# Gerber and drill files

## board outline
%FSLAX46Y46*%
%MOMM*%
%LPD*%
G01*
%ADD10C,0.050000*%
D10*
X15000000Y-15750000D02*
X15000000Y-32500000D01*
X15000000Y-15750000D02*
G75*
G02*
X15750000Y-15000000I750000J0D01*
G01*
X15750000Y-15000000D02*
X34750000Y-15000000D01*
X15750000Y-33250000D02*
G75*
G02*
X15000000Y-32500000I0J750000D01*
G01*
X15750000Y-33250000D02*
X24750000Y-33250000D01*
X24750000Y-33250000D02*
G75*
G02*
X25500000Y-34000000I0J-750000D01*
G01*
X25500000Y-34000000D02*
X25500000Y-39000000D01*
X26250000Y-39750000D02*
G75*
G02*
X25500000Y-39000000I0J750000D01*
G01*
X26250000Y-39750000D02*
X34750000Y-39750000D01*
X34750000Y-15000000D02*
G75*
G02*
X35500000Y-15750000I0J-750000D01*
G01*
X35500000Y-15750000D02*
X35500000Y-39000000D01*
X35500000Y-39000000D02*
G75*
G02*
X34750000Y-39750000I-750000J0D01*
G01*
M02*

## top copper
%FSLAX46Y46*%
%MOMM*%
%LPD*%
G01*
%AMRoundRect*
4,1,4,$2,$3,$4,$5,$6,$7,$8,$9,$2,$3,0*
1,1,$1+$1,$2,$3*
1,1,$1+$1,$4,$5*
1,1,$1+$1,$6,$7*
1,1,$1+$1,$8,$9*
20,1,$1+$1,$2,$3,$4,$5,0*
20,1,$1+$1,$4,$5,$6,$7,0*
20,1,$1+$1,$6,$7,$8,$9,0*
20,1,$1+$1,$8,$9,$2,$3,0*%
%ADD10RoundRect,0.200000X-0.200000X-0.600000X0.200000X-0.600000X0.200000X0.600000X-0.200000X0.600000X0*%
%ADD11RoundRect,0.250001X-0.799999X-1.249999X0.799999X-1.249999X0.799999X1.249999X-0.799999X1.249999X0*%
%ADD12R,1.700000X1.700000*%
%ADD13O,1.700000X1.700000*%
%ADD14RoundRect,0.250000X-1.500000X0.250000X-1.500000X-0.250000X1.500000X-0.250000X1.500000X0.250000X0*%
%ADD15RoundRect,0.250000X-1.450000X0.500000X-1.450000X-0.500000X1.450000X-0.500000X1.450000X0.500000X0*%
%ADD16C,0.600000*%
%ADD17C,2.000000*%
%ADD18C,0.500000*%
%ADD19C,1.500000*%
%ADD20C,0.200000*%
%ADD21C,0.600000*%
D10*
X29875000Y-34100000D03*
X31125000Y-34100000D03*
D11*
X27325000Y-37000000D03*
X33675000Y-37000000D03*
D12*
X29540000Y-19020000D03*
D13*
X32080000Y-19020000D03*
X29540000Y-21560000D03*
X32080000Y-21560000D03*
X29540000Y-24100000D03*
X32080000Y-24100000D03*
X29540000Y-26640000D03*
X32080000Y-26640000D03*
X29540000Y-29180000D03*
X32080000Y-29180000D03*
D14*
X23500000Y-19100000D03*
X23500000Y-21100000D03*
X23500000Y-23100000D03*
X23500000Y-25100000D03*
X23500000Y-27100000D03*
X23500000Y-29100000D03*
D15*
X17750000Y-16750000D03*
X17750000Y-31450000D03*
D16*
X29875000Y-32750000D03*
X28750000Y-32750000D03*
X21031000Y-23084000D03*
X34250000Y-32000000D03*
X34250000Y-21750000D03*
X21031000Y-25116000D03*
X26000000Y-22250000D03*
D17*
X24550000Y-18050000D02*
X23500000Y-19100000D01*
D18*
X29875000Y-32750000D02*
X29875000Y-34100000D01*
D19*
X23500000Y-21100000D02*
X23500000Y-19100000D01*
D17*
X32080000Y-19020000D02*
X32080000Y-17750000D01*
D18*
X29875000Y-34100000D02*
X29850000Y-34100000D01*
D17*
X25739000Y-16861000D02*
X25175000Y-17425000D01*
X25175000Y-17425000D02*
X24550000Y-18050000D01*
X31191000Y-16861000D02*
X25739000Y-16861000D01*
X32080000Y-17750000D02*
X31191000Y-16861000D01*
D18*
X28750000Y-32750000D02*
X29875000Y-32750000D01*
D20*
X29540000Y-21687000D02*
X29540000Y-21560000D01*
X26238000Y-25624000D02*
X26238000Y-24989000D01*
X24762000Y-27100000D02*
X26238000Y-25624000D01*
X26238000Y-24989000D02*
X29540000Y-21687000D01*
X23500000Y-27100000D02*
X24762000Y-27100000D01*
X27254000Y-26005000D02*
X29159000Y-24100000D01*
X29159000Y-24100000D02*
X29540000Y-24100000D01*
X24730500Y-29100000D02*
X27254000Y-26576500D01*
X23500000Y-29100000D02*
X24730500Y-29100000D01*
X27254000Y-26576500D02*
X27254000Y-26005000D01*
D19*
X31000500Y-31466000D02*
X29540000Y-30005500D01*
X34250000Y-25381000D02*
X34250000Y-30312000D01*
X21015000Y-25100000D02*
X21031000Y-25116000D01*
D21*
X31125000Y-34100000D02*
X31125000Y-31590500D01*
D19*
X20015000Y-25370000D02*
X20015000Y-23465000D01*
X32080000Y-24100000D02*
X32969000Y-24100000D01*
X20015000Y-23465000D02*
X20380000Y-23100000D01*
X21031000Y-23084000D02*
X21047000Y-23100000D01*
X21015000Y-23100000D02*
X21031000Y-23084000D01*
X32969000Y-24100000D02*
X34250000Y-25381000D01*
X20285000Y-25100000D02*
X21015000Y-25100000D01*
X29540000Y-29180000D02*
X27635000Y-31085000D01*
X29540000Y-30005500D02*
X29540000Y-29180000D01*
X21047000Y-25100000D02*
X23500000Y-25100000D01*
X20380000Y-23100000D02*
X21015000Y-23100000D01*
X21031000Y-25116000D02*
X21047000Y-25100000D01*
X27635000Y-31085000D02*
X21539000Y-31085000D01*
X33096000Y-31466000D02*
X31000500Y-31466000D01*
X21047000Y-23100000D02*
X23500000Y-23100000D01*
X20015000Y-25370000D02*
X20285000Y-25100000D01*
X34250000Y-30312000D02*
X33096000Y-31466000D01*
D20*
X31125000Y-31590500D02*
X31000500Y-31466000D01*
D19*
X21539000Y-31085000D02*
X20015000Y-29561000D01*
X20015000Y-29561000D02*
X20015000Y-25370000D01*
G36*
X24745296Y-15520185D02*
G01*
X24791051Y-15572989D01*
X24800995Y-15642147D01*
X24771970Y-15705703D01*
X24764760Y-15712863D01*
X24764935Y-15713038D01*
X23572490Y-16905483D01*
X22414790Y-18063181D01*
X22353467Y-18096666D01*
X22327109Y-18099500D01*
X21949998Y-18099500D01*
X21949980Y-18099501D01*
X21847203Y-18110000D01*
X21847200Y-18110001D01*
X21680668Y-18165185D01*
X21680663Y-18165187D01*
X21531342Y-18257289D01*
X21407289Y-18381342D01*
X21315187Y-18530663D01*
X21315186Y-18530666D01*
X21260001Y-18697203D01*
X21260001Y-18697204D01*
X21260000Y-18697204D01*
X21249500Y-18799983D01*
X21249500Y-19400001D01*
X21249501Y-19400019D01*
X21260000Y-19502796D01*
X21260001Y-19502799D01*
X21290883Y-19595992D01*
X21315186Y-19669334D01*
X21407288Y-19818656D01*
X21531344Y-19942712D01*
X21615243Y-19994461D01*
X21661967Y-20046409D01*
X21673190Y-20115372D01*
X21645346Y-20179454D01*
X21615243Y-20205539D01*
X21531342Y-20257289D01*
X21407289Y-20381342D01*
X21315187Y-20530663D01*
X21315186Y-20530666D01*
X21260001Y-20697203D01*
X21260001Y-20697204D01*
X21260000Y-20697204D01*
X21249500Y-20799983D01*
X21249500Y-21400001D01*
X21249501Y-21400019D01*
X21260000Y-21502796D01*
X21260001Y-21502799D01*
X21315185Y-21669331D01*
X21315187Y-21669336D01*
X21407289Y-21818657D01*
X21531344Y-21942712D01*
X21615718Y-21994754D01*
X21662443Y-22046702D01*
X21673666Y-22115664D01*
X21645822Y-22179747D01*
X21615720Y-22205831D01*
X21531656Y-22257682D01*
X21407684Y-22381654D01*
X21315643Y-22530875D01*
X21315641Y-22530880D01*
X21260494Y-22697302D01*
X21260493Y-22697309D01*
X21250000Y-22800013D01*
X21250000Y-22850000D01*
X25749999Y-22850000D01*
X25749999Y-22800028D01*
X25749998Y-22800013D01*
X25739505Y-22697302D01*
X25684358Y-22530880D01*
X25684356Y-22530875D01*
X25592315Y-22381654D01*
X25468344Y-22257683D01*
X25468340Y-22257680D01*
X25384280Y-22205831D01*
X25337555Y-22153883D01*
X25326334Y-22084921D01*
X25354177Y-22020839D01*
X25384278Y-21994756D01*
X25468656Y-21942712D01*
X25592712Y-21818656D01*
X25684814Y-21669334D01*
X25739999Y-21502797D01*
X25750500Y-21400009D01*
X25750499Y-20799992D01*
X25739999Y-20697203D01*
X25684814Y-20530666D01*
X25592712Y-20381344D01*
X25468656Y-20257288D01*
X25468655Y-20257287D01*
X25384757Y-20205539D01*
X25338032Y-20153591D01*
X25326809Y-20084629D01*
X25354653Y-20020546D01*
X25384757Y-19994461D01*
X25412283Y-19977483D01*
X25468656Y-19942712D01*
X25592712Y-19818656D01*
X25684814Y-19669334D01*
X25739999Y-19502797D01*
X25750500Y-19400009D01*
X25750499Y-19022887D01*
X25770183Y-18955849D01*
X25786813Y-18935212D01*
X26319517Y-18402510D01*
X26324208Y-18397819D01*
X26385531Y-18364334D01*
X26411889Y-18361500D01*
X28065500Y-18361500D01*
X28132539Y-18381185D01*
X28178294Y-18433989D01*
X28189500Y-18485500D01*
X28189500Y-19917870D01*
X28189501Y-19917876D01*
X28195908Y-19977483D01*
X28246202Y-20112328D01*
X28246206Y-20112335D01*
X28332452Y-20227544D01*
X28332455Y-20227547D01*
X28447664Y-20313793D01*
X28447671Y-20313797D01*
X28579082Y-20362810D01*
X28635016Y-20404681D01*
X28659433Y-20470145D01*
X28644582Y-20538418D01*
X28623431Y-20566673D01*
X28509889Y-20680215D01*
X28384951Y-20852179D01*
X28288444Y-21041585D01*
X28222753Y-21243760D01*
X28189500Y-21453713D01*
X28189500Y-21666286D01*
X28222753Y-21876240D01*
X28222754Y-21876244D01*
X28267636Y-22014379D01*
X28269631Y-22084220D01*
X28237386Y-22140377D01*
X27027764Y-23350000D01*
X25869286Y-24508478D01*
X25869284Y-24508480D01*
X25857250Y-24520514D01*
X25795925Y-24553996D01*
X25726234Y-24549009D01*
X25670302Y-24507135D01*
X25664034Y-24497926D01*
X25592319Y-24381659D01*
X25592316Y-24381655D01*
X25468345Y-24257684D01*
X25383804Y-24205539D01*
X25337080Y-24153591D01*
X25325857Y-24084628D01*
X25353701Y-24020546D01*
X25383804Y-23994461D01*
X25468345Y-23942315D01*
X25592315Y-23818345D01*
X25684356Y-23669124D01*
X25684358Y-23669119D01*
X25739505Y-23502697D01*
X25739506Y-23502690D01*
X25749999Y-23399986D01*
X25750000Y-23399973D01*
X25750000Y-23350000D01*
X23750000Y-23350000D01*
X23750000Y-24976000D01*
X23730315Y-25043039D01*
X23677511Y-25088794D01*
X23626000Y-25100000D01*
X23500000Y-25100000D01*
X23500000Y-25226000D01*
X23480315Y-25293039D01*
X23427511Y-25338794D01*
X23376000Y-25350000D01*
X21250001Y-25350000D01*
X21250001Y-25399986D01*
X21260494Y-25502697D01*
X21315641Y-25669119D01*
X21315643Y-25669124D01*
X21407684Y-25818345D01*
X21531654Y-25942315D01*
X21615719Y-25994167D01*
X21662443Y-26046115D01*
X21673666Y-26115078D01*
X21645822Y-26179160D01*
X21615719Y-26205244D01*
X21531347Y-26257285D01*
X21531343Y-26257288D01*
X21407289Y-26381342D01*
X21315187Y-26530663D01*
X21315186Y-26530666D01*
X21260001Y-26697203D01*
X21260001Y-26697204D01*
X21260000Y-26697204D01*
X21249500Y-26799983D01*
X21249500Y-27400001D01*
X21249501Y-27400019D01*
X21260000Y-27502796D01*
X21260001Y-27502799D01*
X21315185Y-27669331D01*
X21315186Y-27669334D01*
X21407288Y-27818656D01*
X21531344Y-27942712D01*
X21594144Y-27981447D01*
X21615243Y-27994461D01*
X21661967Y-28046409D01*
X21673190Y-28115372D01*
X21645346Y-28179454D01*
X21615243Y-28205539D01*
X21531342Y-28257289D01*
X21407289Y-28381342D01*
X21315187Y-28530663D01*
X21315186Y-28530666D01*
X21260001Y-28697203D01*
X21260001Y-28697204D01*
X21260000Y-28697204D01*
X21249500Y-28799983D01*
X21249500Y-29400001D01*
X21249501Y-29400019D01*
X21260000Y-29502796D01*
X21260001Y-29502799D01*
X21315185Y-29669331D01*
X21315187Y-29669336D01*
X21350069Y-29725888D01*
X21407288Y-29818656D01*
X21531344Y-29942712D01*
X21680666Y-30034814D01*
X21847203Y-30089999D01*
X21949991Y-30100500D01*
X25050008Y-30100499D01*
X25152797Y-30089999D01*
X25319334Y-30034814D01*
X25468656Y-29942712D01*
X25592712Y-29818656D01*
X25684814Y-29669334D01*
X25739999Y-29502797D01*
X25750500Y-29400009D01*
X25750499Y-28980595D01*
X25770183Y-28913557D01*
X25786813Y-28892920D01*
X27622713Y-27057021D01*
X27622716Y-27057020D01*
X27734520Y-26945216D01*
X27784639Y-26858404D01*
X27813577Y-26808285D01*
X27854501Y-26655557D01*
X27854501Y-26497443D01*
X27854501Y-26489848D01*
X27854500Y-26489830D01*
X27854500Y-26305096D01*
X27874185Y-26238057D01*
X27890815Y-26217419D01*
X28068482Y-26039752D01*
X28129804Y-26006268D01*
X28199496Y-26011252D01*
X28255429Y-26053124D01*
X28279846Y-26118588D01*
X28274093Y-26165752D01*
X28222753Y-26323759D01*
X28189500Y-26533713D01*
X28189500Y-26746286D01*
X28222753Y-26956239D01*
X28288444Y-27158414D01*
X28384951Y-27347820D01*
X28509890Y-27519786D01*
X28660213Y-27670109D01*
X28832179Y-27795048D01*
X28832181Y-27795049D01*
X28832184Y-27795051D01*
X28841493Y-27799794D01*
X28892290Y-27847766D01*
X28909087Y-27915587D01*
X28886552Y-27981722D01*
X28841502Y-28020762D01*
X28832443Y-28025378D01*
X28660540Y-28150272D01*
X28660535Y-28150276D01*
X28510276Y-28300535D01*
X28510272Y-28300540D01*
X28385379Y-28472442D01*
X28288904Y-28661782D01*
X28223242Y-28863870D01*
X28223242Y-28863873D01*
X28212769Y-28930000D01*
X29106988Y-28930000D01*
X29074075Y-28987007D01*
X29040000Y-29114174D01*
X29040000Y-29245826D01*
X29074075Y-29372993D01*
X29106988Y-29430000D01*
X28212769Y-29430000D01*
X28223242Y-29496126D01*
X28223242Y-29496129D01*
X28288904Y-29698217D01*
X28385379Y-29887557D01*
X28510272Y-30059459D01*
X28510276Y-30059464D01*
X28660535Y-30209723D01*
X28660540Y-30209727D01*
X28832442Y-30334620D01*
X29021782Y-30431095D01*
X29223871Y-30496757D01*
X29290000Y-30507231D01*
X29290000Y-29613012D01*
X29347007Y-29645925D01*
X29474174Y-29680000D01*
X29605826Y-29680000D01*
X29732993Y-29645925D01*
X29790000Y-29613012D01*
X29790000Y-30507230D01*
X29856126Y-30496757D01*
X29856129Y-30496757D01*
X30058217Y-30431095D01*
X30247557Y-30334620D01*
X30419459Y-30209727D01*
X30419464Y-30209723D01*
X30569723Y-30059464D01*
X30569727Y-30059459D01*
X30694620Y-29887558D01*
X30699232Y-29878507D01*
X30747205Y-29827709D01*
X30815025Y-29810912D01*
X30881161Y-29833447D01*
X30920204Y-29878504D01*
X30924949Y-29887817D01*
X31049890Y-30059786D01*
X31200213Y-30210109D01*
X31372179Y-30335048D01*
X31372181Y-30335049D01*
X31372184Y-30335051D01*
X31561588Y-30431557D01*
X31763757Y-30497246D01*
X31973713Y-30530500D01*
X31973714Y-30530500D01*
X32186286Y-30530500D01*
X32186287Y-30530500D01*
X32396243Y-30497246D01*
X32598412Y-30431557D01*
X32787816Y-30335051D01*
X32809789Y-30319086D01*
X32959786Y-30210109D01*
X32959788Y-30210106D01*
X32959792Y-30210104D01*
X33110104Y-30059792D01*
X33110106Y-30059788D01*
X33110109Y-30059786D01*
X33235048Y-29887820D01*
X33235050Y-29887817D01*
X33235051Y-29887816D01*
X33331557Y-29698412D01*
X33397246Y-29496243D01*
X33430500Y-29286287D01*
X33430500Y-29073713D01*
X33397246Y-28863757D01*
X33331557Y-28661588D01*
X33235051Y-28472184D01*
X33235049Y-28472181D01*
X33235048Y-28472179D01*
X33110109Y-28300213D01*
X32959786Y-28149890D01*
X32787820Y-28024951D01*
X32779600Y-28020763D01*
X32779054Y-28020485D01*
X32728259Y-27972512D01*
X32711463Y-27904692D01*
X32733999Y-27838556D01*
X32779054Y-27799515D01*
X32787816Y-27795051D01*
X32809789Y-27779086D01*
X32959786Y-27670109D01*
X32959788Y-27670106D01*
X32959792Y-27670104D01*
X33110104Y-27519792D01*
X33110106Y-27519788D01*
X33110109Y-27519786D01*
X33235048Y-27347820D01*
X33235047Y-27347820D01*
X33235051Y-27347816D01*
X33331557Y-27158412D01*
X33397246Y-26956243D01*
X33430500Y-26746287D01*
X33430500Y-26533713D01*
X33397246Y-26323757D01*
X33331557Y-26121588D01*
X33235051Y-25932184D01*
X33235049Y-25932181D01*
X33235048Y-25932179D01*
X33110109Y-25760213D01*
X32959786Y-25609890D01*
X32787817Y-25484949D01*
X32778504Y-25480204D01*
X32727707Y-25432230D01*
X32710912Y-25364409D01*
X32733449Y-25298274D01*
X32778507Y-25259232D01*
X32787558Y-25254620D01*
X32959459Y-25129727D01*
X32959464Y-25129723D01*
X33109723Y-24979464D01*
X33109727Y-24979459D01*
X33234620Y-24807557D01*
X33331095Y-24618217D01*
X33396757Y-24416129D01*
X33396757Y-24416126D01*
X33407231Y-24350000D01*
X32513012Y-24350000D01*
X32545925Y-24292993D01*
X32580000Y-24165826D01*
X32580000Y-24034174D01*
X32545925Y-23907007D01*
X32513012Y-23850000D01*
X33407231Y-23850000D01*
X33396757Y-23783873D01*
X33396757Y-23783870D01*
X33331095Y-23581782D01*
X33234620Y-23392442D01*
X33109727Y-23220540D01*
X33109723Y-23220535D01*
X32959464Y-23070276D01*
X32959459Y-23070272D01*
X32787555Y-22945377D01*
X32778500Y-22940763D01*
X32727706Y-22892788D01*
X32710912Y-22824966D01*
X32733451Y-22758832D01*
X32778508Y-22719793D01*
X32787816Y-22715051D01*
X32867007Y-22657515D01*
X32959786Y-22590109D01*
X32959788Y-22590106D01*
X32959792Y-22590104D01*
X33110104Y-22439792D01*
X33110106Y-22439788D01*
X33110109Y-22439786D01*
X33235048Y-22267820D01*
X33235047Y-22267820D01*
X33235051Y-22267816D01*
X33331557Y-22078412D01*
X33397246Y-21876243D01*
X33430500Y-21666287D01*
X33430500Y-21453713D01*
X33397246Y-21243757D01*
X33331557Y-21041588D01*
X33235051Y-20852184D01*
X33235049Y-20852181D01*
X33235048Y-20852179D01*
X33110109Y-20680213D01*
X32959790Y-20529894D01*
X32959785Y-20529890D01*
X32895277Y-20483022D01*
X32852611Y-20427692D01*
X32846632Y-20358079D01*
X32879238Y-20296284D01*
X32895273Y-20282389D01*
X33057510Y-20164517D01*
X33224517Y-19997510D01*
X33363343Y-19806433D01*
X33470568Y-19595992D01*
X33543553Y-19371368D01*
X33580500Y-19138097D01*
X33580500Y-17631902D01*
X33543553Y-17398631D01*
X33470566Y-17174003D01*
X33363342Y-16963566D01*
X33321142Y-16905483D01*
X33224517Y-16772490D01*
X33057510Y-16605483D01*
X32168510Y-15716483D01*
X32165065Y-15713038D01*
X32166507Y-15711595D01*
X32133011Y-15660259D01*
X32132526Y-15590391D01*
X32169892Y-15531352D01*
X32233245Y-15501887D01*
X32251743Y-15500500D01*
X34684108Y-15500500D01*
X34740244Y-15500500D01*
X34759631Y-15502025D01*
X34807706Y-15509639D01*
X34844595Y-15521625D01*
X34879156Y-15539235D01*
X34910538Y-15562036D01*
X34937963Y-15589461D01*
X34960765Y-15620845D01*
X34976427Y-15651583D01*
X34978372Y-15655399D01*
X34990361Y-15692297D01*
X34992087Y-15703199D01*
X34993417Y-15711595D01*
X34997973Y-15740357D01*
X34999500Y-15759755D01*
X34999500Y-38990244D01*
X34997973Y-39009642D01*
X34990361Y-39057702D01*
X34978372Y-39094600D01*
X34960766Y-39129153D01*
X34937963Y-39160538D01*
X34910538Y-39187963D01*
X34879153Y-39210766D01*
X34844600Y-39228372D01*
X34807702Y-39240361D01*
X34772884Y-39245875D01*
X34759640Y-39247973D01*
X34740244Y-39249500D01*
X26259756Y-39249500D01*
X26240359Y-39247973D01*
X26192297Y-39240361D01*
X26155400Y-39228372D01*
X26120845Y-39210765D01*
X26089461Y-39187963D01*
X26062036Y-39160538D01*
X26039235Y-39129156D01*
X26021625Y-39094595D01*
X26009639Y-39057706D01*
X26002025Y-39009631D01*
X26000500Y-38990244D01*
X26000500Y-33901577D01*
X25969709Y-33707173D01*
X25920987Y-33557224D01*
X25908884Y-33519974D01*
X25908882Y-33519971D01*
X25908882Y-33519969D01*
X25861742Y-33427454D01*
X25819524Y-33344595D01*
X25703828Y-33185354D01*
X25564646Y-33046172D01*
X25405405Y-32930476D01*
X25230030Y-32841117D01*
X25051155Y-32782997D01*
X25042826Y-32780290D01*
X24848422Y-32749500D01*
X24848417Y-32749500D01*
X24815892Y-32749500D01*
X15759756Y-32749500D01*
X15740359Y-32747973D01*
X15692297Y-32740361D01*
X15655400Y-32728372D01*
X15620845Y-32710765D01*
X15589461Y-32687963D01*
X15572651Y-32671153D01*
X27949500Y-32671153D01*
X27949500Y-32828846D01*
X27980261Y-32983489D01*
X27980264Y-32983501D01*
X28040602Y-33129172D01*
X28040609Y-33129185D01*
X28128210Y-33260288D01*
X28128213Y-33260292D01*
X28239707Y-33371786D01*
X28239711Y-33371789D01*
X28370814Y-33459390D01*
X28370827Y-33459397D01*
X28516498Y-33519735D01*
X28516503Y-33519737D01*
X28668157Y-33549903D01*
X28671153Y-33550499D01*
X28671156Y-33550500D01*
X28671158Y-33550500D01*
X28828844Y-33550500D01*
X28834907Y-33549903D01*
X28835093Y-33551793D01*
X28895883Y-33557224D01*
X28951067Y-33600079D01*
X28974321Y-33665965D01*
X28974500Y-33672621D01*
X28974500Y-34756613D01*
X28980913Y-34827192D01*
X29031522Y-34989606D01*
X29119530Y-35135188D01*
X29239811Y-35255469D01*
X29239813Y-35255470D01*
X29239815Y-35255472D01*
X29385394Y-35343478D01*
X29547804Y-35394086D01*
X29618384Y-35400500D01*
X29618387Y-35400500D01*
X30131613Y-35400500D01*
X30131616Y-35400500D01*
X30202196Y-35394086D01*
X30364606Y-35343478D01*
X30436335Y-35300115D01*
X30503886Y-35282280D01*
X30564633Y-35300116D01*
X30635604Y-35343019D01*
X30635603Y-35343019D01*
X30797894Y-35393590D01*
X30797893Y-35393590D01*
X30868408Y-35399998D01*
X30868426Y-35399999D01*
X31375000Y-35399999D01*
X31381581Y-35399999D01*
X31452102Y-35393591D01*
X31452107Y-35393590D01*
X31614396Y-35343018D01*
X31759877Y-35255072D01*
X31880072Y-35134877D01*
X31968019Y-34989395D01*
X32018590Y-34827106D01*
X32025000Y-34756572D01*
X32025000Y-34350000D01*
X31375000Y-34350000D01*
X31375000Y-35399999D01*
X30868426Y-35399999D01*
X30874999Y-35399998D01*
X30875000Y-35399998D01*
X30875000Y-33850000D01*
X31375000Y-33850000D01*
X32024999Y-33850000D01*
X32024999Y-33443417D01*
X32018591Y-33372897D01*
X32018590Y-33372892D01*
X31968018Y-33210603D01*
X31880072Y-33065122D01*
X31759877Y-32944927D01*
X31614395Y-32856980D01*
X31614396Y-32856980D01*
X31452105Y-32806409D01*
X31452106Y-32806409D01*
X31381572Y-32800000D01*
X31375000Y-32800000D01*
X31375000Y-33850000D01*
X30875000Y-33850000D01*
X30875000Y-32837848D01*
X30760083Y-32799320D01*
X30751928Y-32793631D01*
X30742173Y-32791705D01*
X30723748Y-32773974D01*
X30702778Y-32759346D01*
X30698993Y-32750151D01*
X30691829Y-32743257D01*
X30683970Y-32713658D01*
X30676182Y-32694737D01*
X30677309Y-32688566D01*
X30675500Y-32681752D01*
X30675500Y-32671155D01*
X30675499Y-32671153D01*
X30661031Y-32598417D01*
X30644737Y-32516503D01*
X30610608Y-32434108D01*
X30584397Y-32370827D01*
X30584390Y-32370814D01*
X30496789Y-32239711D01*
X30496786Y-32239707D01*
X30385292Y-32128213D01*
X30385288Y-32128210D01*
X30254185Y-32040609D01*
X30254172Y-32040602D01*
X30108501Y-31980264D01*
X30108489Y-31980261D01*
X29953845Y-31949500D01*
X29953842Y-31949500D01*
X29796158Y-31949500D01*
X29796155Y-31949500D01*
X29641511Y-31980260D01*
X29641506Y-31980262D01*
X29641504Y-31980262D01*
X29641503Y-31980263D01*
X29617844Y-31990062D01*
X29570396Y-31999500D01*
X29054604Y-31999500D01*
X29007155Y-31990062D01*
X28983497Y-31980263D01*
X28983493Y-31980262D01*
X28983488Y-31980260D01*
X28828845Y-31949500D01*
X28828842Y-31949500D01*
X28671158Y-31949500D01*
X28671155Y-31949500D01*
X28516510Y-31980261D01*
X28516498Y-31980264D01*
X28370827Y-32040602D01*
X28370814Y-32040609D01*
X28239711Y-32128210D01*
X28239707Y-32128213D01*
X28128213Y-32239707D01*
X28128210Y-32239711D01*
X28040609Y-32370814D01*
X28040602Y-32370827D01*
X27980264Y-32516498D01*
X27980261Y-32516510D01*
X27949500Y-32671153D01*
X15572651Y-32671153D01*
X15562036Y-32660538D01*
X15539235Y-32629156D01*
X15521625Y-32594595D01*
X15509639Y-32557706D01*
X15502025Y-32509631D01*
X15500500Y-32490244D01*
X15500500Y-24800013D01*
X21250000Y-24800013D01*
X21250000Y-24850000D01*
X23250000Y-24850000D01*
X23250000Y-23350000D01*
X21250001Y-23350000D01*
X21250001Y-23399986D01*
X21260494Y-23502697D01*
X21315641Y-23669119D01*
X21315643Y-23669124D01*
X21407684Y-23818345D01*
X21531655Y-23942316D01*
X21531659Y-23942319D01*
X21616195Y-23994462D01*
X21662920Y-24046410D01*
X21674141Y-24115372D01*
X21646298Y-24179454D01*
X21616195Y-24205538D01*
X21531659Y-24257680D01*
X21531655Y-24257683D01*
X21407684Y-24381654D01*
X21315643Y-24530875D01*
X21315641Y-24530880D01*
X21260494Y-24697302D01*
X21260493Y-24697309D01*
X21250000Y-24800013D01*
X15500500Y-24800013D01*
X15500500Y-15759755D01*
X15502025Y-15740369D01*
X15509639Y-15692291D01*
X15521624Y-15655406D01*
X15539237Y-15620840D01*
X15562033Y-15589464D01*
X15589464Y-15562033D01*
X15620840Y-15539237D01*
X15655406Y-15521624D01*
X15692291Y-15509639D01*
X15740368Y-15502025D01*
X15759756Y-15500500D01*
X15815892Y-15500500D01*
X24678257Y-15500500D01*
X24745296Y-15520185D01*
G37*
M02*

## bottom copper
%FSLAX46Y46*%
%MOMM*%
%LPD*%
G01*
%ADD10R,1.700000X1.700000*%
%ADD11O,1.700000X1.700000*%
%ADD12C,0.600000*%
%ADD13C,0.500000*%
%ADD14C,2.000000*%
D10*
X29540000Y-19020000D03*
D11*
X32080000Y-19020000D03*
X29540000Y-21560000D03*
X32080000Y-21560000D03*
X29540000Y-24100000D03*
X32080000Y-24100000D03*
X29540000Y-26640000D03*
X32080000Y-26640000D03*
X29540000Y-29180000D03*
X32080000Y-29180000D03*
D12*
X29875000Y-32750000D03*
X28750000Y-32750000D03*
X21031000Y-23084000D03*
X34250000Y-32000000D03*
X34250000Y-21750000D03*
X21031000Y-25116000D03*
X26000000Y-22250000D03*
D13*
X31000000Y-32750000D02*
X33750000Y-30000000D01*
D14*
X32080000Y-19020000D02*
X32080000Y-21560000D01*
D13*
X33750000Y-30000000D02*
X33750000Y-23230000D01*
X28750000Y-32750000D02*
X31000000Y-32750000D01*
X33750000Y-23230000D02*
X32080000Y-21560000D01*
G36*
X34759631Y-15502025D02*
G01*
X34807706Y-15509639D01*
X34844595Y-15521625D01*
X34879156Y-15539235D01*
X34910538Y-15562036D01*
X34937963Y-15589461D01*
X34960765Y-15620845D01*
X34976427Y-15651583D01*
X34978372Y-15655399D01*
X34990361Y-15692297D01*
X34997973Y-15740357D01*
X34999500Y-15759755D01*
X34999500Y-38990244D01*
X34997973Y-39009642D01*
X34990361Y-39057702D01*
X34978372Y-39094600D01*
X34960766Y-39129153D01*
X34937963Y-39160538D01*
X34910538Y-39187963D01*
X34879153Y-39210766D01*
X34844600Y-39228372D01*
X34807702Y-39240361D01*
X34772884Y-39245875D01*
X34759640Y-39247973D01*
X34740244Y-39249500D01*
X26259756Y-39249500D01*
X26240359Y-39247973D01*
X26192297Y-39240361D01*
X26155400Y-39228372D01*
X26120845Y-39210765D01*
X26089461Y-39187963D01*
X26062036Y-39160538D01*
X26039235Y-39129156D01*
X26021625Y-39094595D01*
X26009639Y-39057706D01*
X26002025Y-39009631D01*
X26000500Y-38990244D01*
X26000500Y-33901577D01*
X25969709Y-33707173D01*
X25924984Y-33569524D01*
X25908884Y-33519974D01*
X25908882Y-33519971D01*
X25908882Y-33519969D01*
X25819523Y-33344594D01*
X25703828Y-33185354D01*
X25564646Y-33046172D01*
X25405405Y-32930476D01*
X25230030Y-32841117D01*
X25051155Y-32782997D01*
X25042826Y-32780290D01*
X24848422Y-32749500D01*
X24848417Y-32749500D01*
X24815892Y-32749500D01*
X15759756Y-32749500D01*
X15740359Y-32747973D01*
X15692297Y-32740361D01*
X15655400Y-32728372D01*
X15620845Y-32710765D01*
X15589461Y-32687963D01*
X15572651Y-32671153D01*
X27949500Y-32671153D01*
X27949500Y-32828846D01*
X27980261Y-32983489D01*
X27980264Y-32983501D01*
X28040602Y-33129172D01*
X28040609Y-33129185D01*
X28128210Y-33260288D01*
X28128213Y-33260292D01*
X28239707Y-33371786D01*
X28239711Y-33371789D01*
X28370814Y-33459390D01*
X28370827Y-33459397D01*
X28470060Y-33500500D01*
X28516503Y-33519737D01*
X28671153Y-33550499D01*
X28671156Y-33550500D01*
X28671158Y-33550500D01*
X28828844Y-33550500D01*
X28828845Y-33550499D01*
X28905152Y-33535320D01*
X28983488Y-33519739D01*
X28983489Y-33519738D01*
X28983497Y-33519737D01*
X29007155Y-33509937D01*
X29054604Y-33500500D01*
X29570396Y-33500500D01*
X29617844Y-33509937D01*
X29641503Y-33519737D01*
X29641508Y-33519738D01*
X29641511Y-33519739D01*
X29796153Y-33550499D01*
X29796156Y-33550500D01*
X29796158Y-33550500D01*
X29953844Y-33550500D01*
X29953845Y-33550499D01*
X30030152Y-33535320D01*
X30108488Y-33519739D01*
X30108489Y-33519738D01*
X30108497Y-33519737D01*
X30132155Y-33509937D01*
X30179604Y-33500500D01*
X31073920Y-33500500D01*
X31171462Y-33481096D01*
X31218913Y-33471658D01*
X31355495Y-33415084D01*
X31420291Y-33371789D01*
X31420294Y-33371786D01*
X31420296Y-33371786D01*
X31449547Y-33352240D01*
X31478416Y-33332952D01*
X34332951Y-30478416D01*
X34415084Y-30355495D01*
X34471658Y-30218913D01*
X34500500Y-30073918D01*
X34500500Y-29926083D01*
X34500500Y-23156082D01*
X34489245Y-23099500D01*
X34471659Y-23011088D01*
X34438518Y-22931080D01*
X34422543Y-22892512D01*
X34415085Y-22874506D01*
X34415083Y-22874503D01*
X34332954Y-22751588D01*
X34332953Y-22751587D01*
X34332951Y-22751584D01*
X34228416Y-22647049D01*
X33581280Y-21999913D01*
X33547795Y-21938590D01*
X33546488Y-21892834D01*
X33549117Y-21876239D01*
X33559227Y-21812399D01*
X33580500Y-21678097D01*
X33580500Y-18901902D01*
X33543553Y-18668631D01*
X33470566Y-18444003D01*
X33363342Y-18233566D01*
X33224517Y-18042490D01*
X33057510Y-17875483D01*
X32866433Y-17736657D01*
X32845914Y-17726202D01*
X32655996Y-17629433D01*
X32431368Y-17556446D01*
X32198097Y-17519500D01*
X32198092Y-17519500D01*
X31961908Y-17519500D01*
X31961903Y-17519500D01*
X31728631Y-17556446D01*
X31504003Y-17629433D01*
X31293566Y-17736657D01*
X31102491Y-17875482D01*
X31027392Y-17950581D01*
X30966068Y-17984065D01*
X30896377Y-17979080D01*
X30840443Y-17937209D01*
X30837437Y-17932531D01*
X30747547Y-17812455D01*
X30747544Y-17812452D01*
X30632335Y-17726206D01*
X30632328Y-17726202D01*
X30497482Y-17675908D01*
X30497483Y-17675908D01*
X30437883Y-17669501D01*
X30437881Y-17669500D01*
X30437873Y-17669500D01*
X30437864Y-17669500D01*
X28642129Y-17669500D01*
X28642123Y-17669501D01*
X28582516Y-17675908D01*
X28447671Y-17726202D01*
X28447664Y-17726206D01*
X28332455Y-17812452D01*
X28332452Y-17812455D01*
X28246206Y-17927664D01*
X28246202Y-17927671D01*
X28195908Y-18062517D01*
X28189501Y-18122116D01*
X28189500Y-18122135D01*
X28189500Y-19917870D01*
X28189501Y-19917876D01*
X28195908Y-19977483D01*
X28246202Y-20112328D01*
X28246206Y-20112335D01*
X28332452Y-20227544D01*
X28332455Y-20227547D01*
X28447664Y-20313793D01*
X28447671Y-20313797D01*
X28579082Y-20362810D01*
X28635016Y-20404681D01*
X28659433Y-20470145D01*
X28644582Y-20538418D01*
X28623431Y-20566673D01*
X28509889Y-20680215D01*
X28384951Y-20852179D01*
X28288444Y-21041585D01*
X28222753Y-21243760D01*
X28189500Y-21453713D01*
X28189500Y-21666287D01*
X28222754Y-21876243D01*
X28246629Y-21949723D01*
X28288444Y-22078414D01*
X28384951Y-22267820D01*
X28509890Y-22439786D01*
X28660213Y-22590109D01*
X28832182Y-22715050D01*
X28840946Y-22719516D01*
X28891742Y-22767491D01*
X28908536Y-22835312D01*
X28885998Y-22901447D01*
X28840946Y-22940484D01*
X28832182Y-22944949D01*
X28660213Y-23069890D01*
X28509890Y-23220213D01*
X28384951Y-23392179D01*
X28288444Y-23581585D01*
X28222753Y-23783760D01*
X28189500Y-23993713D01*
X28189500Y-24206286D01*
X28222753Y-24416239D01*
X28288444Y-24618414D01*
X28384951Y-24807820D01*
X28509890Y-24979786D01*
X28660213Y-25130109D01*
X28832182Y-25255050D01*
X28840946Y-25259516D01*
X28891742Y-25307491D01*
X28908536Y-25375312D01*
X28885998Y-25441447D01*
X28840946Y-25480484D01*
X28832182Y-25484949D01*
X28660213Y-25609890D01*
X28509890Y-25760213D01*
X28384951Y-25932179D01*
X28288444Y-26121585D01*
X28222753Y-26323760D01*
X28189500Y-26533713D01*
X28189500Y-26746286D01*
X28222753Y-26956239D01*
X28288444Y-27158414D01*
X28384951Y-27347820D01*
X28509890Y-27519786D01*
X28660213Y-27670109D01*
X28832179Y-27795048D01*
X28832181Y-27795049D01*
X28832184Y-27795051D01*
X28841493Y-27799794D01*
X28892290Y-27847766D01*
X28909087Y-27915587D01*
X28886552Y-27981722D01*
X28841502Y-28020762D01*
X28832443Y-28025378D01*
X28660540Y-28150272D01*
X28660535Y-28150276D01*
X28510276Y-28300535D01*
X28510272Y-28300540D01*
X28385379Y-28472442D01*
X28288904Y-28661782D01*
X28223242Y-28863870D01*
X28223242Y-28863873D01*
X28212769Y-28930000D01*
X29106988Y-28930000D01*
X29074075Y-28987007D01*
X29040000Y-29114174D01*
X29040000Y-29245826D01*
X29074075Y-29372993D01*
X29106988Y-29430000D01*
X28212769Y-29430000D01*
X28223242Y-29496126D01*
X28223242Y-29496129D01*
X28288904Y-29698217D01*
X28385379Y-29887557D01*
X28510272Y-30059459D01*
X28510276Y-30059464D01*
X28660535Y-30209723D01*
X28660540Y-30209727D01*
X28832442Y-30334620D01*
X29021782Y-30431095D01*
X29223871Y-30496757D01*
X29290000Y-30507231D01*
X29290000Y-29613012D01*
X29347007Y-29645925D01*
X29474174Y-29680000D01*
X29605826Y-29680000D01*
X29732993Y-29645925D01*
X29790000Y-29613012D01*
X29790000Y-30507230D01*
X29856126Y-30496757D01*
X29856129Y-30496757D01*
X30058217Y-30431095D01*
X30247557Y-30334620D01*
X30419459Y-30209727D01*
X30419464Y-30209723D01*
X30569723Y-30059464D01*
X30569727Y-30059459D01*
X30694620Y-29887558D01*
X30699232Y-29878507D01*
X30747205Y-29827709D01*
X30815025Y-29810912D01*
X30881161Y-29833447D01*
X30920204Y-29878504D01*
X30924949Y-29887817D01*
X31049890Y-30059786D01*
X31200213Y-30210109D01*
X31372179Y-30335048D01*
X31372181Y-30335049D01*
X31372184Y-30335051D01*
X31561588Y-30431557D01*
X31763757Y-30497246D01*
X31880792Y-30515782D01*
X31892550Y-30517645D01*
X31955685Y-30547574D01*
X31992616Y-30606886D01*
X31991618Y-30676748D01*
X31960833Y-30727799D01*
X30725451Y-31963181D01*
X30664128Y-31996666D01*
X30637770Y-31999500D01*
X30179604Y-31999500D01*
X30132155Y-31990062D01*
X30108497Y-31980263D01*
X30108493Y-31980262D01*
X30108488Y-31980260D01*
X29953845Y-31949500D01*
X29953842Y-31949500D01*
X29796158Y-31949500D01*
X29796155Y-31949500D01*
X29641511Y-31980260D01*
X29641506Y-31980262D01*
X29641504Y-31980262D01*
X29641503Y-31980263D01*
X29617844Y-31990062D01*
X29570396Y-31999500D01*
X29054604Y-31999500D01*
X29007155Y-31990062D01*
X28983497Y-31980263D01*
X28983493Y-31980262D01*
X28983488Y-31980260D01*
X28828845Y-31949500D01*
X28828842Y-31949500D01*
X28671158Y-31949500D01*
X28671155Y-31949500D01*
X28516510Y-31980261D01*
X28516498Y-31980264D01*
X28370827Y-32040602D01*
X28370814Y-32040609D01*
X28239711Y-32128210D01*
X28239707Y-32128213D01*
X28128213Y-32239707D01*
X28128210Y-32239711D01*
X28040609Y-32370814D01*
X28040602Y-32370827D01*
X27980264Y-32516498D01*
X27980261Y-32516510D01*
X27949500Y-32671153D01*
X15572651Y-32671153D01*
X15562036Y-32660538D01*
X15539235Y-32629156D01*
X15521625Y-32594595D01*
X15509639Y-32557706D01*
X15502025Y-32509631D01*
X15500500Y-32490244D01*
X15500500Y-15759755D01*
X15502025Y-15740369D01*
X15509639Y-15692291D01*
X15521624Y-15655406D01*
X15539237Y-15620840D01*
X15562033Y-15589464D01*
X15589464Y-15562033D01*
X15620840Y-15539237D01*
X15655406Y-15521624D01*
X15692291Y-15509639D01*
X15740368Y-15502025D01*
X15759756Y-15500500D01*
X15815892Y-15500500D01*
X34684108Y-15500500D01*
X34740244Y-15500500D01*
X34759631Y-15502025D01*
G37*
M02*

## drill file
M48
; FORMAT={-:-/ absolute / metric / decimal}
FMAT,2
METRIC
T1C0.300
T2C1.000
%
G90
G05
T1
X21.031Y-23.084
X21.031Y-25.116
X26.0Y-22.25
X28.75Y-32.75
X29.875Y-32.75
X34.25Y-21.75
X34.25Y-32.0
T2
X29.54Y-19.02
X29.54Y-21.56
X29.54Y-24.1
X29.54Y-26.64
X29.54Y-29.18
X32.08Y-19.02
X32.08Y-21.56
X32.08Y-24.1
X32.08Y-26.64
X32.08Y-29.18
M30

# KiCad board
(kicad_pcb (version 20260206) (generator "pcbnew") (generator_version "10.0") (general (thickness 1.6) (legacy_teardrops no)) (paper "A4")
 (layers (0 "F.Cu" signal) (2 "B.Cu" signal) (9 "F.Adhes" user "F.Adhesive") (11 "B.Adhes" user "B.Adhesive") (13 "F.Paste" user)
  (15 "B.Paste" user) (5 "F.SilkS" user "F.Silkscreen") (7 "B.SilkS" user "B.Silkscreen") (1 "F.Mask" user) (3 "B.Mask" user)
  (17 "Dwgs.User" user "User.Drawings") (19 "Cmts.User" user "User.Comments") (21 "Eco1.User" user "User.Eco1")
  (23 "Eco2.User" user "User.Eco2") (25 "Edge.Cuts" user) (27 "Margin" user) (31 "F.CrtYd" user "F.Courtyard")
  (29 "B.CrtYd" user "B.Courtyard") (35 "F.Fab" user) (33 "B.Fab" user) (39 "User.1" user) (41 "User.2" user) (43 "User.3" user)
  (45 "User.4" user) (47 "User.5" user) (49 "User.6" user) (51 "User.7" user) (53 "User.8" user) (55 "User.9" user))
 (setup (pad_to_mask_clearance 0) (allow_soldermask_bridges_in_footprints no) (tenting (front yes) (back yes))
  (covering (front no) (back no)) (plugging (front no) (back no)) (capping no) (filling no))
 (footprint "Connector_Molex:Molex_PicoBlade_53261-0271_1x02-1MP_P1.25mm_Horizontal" (layer "F.Cu") (at 30.5 36.5)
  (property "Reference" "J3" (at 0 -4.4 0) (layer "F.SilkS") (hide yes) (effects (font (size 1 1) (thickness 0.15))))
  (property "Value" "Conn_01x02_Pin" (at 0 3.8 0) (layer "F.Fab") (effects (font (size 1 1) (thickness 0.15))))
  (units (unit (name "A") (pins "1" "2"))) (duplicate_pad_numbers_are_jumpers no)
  (pad "1" smd roundrect (at -0.625 -2.4) (size 0.8 1.6) (layers "F.Cu" "F.Mask" "F.Paste") (roundrect_rratio 0.25) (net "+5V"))
  (pad "2" smd roundrect (at 0.625 -2.4) (size 0.8 1.6) (layers "F.Cu" "F.Mask" "F.Paste") (roundrect_rratio 0.25) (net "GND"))
  (pad "MP" smd roundrect (at -3.175 0.5) (size 2.1 3) (layers "F.Cu" "F.Mask" "F.Paste") (roundrect_rratio 0.119048) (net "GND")
   (zone_connect 2))
  (pad "MP" smd roundrect (at 3.175 0.5) (size 2.1 3) (layers "F.Cu" "F.Mask" "F.Paste") (roundrect_rratio 0.119048) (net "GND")
   (zone_connect 2)))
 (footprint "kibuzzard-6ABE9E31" (layer "F.Cu") (at 26.5 24 90)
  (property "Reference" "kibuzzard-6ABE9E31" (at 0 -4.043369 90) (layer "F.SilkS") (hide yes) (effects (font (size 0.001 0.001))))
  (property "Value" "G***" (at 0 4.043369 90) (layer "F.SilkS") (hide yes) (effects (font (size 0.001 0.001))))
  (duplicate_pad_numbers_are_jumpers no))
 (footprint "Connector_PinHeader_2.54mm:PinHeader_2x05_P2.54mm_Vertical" (layer "F.Cu") (at 29.54 19.02)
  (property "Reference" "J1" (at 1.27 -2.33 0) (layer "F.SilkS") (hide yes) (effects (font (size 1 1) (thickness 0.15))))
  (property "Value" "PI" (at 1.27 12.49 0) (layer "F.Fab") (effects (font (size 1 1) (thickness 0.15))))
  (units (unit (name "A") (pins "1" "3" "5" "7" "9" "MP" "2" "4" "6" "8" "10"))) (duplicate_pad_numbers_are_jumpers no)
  (pad "1" thru_hole rect (at 0 0) (size 1.7 1.7) (drill 1) (layers "*.Cu" "*.Mask") (remove_unused_layers no)
   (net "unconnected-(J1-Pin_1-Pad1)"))
  (pad "2" thru_hole oval (at 2.54 0) (size 1.7 1.7) (drill 1) (layers "*.Cu" "*.Mask") (remove_unused_layers no) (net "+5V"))
  (pad "3" thru_hole oval (at 0 2.54) (size 1.7 1.7) (drill 1) (layers "*.Cu" "*.Mask") (remove_unused_layers no) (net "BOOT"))
  (pad "4" thru_hole oval (at 2.54 2.54) (size 1.7 1.7) (drill 1) (layers "*.Cu" "*.Mask") (remove_unused_layers no) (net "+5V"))
  (pad "5" thru_hole oval (at 0 5.08) (size 1.7 1.7) (drill 1) (layers "*.Cu" "*.Mask") (remove_unused_layers no) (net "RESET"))
  (pad "6" thru_hole oval (at 2.54 5.08) (size 1.7 1.7) (drill 1) (layers "*.Cu" "*.Mask") (remove_unused_layers no) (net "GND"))
  (pad "7" thru_hole oval (at 0 7.62) (size 1.7 1.7) (drill 1) (layers "*.Cu" "*.Mask") (remove_unused_layers no)
   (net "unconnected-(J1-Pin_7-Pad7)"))
  (pad "8" thru_hole oval (at 2.54 7.62) (size 1.7 1.7) (drill 1) (layers "*.Cu" "*.Mask") (remove_unused_layers no)
   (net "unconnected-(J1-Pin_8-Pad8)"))
  (pad "9" thru_hole oval (at 0 10.16) (size 1.7 1.7) (drill 1) (layers "*.Cu" "*.Mask") (remove_unused_layers no) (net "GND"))
  (pad "10" thru_hole oval (at 2.54 10.16) (size 1.7 1.7) (drill 1) (layers "*.Cu" "*.Mask") (remove_unused_layers no)
   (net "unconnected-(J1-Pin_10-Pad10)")))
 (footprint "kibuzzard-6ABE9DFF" (layer "F.Cu") (at 33.75 33.25 90)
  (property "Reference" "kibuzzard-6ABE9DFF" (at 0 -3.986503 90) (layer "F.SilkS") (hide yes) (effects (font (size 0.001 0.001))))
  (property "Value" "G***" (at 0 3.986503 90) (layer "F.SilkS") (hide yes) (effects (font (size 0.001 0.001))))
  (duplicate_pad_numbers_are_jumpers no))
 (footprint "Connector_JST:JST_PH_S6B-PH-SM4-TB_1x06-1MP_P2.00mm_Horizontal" (layer "F.Cu") (at 20.65 24.1 -90)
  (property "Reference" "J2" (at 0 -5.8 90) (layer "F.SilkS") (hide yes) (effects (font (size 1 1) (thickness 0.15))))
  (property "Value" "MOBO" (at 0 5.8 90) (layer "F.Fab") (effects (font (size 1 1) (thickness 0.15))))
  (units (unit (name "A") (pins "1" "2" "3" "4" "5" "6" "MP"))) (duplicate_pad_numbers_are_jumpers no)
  (pad "1" smd roundrect (at -5 -2.85 270) (size 1 3.5) (layers "F.Cu" "F.Mask" "F.Paste") (roundrect_rratio 0.25) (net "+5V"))
  (pad "2" smd roundrect (at -3 -2.85 270) (size 1 3.5) (layers "F.Cu" "F.Mask" "F.Paste") (roundrect_rratio 0.25) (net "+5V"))
  (pad "3" smd roundrect (at -1 -2.85 270) (size 1 3.5) (layers "F.Cu" "F.Mask" "F.Paste") (roundrect_rratio 0.25) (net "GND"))
  (pad "4" smd roundrect (at 1 -2.85 270) (size 1 3.5) (layers "F.Cu" "F.Mask" "F.Paste") (roundrect_rratio 0.25) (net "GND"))
  (pad "5" smd roundrect (at 3 -2.85 270) (size 1 3.5) (layers "F.Cu" "F.Mask" "F.Paste") (roundrect_rratio 0.25) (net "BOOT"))
  (pad "6" smd roundrect (at 5 -2.85 270) (size 1 3.5) (layers "F.Cu" "F.Mask" "F.Paste") (roundrect_rratio 0.25) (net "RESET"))
  (pad "MP" smd roundrect (at -7.35 2.9 270) (size 1.5 3.4) (layers "F.Cu" "F.Mask" "F.Paste") (roundrect_rratio 0.1666666667) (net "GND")
   (zone_connect 2))
  (pad "MP" smd roundrect (at 7.35 2.9 270) (size 1.5 3.4) (layers "F.Cu" "F.Mask" "F.Paste") (roundrect_rratio 0.1666666667) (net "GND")
   (zone_connect 2)))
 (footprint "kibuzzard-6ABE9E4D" (layer "F.Cu") (at 34.4 24.1 90)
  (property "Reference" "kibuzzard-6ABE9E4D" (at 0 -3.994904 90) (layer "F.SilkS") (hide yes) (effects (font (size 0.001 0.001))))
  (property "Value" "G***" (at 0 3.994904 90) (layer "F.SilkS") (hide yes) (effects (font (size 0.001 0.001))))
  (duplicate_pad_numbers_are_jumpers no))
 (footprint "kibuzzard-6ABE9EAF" (layer "B.Cu") (at 21.2 29.8 90)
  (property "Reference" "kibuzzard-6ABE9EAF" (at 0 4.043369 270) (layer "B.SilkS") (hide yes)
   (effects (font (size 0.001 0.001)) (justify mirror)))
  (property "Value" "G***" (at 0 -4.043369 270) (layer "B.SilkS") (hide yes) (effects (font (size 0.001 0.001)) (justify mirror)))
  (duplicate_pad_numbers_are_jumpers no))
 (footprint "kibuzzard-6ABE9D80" (layer "B.Cu") (at 23.6 28.1 90)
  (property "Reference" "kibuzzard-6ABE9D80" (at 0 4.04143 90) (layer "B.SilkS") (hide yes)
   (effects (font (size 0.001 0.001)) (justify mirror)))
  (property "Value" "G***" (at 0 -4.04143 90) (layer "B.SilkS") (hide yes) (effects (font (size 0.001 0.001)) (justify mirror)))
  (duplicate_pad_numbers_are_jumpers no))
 (gr_line (start 15 15.75) (end 15 32.5) (stroke (width 0.05) (type default)) (layer "Edge.Cuts"))
 (gr_arc (start 15 15.75) (mid 15.21967 15.21967) (end 15.75 15) (stroke (width 0.05) (type default)) (layer "Edge.Cuts"))
 (gr_line (start 15.75 15) (end 34.75 15) (stroke (width 0.05) (type default)) (layer "Edge.Cuts"))
 (gr_arc (start 15.75 33.25) (mid 15.21967 33.03033) (end 15 32.5) (stroke (width 0.05) (type default)) (layer "Edge.Cuts"))
 (gr_line (start 15.75 33.25) (end 24.75 33.25) (stroke (width 0.05) (type default)) (layer "Edge.Cuts"))
 (gr_arc (start 24.75 33.25) (mid 25.28033 33.46967) (end 25.5 34) (stroke (width 0.05) (type default)) (layer "Edge.Cuts"))
 (gr_line (start 25.5 34) (end 25.5 39) (stroke (width 0.05) (type default)) (layer "Edge.Cuts"))
 (gr_arc (start 26.25 39.75) (mid 25.71967 39.53033) (end 25.5 39) (stroke (width 0.05) (type default)) (layer "Edge.Cuts"))
 (gr_line (start 26.25 39.75) (end 34.75 39.75) (stroke (width 0.05) (type default)) (layer "Edge.Cuts"))
 (gr_arc (start 34.75 15) (mid 35.28033 15.21967) (end 35.5 15.75) (stroke (width 0.05) (type default)) (layer "Edge.Cuts"))
 (gr_line (start 35.5 15.75) (end 35.5 39) (stroke (width 0.05) (type default)) (layer "Edge.Cuts"))
 (gr_arc (start 35.5 39) (mid 35.28033 39.53033) (end 34.75 39.75) (stroke (width 0.05) (type default)) (layer "Edge.Cuts"))
 (segment (start 24.55 18.05) (end 23.5 19.1) (width 2) (layer "F.Cu") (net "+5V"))
 (segment (start 29.875 32.75) (end 29.875 34.1) (width 0.5) (layer "F.Cu") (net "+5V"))
 (segment (start 23.5 21.1) (end 23.5 19.1) (width 1.5) (layer "F.Cu") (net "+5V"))
 (segment (start 32.08 19.02) (end 32.08 17.75) (width 2) (layer "F.Cu") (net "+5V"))
 (segment (start 29.875 34.1) (end 29.85 34.1) (width 0.5) (layer "F.Cu") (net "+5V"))
 (segment (start 25.739 16.861) (end 25.175 17.425) (width 2) (layer "F.Cu") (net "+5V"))
 (segment (start 25.175 17.425) (end 24.55 18.05) (width 2) (layer "F.Cu") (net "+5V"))
 (segment (start 31.191 16.861) (end 25.739 16.861) (width 2) (layer "F.Cu") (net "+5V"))
 (segment (start 32.08 17.75) (end 31.191 16.861) (width 2) (layer "F.Cu") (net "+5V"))
 (segment (start 28.75 32.75) (end 29.875 32.75) (width 0.5) (layer "F.Cu") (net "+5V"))
 (via (at 29.875 32.75) (size 0.6) (drill 0.3) (layers "F.Cu" "B.Cu") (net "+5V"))
 (via (at 28.75 32.75) (size 0.6) (drill 0.3) (layers "F.Cu" "B.Cu") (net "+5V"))
 (segment (start 31 32.75) (end 33.75 30) (width 0.5) (layer "B.Cu") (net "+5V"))
 (segment (start 32.08 19.02) (end 32.08 21.56) (width 2) (layer "B.Cu") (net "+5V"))
 (segment (start 33.75 30) (end 33.75 23.23) (width 0.5) (layer "B.Cu") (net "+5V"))
 (segment (start 28.75 32.75) (end 31 32.75) (width 0.5) (layer "B.Cu") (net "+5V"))
 (segment (start 33.75 23.23) (end 32.08 21.56) (width 0.5) (layer "B.Cu") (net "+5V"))
 (segment (start 29.54 21.687) (end 29.54 21.56) (width 0.2) (layer "F.Cu") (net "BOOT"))
 (segment (start 26.238 25.624) (end 26.238 24.989) (width 0.2) (layer "F.Cu") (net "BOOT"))
 (segment (start 24.762 27.1) (end 26.238 25.624) (width 0.2) (layer "F.Cu") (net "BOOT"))
 (segment (start 26.238 24.989) (end 29.54 21.687) (width 0.2) (layer "F.Cu") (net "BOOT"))
 (segment (start 23.5 27.1) (end 24.762 27.1) (width 0.2) (layer "F.Cu") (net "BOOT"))
 (segment (start 27.254 26.005) (end 29.159 24.1) (width 0.2) (layer "F.Cu") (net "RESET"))
 (segment (start 29.159 24.1) (end 29.54 24.1) (width 0.2) (layer "F.Cu") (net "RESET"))
 (segment (start 24.7305 29.1) (end 27.254 26.5765) (width 0.2) (layer "F.Cu") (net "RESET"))
 (segment (start 23.5 29.1) (end 24.7305 29.1) (width 0.2) (layer "F.Cu") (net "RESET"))
 (segment (start 27.254 26.5765) (end 27.254 26.005) (width 0.2) (layer "F.Cu") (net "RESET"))
 (segment (start 31.0005 31.466) (end 29.54 30.0055) (width 1.5) (layer "F.Cu") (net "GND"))
 (segment (start 34.25 25.381) (end 34.25 30.312) (width 1.5) (layer "F.Cu") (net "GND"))
 (segment (start 21.015 25.1) (end 21.031 25.116) (width 1.5) (layer "F.Cu") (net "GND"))
 (segment (start 31.125 34.1) (end 31.125 31.5905) (width 0.6) (layer "F.Cu") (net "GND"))
 (segment (start 20.015 25.37) (end 20.015 23.465) (width 1.5) (layer "F.Cu") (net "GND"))
 (segment (start 32.08 24.1) (end 32.969 24.1) (width 1.5) (layer "F.Cu") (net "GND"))
 (segment (start 20.015 23.465) (end 20.38 23.1) (width 1.5) (layer "F.Cu") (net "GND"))
 (segment (start 21.031 23.084) (end 21.047 23.1) (width 1.5) (layer "F.Cu") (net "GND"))
 (segment (start 21.015 23.1) (end 21.031 23.084) (width 1.5) (layer "F.Cu") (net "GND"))
 (segment (start 32.969 24.1) (end 34.25 25.381) (width 1.5) (layer "F.Cu") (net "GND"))
 (segment (start 20.285 25.1) (end 21.015 25.1) (width 1.5) (layer "F.Cu") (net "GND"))
 (segment (start 29.54 29.18) (end 27.635 31.085) (width 1.5) (layer "F.Cu") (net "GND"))
 (segment (start 29.54 30.0055) (end 29.54 29.18) (width 1.5) (layer "F.Cu") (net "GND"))
 (segment (start 21.047 25.1) (end 23.5 25.1) (width 1.5) (layer "F.Cu") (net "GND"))
 (segment (start 20.38 23.1) (end 21.015 23.1) (width 1.5) (layer "F.Cu") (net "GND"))
 (segment (start 21.031 25.116) (end 21.047 25.1) (width 1.5) (layer "F.Cu") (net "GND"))
 (segment (start 27.635 31.085) (end 21.539 31.085) (width 1.5) (layer "F.Cu") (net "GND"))
 (segment (start 33.096 31.466) (end 31.0005 31.466) (width 1.5) (layer "F.Cu") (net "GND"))
 (segment (start 21.047 23.1) (end 23.5 23.1) (width 1.5) (layer "F.Cu") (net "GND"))
 (segment (start 20.015 25.37) (end 20.285 25.1) (width 1.5) (layer "F.Cu") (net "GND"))
 (segment (start 34.25 30.312) (end 33.096 31.466) (width 1.5) (layer "F.Cu") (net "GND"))
 (segment (start 31.125 31.5905) (end 31.0005 31.466) (width 0.2) (layer "F.Cu") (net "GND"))
 (segment (start 21.539 31.085) (end 20.015 29.561) (width 1.5) (layer "F.Cu") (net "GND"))
 (segment (start 20.015 29.561) (end 20.015 25.37) (width 1.5) (layer "F.Cu") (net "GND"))
 (via (at 21.031 23.084) (size 0.6) (drill 0.3) (layers "F.Cu" "B.Cu") (capping no) (covering (front no) (back no))
  (plugging (front no) (back no)) (filling no) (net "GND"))
 (via (at 34.25 32) (size 0.6) (drill 0.3) (layers "F.Cu" "B.Cu") (free yes) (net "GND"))
 (via (at 34.25 21.75) (size 0.6) (drill 0.3) (layers "F.Cu" "B.Cu") (free yes) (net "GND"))
 (via (at 21.031 25.116) (size 0.6) (drill 0.3) (layers "F.Cu" "B.Cu") (capping no) (covering (front no) (back no))
  (plugging (front no) (back no)) (filling no) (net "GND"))
 (via (at 26 22.25) (size 0.6) (drill 0.3) (layers "F.Cu" "B.Cu") (free yes) (capping no) (covering (front no) (back no))
  (plugging (front no) (back no)) (filling no) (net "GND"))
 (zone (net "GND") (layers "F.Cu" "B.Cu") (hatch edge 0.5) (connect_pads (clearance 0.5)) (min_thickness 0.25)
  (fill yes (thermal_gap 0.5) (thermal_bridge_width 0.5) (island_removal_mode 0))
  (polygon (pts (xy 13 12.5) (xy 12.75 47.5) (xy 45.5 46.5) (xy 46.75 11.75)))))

